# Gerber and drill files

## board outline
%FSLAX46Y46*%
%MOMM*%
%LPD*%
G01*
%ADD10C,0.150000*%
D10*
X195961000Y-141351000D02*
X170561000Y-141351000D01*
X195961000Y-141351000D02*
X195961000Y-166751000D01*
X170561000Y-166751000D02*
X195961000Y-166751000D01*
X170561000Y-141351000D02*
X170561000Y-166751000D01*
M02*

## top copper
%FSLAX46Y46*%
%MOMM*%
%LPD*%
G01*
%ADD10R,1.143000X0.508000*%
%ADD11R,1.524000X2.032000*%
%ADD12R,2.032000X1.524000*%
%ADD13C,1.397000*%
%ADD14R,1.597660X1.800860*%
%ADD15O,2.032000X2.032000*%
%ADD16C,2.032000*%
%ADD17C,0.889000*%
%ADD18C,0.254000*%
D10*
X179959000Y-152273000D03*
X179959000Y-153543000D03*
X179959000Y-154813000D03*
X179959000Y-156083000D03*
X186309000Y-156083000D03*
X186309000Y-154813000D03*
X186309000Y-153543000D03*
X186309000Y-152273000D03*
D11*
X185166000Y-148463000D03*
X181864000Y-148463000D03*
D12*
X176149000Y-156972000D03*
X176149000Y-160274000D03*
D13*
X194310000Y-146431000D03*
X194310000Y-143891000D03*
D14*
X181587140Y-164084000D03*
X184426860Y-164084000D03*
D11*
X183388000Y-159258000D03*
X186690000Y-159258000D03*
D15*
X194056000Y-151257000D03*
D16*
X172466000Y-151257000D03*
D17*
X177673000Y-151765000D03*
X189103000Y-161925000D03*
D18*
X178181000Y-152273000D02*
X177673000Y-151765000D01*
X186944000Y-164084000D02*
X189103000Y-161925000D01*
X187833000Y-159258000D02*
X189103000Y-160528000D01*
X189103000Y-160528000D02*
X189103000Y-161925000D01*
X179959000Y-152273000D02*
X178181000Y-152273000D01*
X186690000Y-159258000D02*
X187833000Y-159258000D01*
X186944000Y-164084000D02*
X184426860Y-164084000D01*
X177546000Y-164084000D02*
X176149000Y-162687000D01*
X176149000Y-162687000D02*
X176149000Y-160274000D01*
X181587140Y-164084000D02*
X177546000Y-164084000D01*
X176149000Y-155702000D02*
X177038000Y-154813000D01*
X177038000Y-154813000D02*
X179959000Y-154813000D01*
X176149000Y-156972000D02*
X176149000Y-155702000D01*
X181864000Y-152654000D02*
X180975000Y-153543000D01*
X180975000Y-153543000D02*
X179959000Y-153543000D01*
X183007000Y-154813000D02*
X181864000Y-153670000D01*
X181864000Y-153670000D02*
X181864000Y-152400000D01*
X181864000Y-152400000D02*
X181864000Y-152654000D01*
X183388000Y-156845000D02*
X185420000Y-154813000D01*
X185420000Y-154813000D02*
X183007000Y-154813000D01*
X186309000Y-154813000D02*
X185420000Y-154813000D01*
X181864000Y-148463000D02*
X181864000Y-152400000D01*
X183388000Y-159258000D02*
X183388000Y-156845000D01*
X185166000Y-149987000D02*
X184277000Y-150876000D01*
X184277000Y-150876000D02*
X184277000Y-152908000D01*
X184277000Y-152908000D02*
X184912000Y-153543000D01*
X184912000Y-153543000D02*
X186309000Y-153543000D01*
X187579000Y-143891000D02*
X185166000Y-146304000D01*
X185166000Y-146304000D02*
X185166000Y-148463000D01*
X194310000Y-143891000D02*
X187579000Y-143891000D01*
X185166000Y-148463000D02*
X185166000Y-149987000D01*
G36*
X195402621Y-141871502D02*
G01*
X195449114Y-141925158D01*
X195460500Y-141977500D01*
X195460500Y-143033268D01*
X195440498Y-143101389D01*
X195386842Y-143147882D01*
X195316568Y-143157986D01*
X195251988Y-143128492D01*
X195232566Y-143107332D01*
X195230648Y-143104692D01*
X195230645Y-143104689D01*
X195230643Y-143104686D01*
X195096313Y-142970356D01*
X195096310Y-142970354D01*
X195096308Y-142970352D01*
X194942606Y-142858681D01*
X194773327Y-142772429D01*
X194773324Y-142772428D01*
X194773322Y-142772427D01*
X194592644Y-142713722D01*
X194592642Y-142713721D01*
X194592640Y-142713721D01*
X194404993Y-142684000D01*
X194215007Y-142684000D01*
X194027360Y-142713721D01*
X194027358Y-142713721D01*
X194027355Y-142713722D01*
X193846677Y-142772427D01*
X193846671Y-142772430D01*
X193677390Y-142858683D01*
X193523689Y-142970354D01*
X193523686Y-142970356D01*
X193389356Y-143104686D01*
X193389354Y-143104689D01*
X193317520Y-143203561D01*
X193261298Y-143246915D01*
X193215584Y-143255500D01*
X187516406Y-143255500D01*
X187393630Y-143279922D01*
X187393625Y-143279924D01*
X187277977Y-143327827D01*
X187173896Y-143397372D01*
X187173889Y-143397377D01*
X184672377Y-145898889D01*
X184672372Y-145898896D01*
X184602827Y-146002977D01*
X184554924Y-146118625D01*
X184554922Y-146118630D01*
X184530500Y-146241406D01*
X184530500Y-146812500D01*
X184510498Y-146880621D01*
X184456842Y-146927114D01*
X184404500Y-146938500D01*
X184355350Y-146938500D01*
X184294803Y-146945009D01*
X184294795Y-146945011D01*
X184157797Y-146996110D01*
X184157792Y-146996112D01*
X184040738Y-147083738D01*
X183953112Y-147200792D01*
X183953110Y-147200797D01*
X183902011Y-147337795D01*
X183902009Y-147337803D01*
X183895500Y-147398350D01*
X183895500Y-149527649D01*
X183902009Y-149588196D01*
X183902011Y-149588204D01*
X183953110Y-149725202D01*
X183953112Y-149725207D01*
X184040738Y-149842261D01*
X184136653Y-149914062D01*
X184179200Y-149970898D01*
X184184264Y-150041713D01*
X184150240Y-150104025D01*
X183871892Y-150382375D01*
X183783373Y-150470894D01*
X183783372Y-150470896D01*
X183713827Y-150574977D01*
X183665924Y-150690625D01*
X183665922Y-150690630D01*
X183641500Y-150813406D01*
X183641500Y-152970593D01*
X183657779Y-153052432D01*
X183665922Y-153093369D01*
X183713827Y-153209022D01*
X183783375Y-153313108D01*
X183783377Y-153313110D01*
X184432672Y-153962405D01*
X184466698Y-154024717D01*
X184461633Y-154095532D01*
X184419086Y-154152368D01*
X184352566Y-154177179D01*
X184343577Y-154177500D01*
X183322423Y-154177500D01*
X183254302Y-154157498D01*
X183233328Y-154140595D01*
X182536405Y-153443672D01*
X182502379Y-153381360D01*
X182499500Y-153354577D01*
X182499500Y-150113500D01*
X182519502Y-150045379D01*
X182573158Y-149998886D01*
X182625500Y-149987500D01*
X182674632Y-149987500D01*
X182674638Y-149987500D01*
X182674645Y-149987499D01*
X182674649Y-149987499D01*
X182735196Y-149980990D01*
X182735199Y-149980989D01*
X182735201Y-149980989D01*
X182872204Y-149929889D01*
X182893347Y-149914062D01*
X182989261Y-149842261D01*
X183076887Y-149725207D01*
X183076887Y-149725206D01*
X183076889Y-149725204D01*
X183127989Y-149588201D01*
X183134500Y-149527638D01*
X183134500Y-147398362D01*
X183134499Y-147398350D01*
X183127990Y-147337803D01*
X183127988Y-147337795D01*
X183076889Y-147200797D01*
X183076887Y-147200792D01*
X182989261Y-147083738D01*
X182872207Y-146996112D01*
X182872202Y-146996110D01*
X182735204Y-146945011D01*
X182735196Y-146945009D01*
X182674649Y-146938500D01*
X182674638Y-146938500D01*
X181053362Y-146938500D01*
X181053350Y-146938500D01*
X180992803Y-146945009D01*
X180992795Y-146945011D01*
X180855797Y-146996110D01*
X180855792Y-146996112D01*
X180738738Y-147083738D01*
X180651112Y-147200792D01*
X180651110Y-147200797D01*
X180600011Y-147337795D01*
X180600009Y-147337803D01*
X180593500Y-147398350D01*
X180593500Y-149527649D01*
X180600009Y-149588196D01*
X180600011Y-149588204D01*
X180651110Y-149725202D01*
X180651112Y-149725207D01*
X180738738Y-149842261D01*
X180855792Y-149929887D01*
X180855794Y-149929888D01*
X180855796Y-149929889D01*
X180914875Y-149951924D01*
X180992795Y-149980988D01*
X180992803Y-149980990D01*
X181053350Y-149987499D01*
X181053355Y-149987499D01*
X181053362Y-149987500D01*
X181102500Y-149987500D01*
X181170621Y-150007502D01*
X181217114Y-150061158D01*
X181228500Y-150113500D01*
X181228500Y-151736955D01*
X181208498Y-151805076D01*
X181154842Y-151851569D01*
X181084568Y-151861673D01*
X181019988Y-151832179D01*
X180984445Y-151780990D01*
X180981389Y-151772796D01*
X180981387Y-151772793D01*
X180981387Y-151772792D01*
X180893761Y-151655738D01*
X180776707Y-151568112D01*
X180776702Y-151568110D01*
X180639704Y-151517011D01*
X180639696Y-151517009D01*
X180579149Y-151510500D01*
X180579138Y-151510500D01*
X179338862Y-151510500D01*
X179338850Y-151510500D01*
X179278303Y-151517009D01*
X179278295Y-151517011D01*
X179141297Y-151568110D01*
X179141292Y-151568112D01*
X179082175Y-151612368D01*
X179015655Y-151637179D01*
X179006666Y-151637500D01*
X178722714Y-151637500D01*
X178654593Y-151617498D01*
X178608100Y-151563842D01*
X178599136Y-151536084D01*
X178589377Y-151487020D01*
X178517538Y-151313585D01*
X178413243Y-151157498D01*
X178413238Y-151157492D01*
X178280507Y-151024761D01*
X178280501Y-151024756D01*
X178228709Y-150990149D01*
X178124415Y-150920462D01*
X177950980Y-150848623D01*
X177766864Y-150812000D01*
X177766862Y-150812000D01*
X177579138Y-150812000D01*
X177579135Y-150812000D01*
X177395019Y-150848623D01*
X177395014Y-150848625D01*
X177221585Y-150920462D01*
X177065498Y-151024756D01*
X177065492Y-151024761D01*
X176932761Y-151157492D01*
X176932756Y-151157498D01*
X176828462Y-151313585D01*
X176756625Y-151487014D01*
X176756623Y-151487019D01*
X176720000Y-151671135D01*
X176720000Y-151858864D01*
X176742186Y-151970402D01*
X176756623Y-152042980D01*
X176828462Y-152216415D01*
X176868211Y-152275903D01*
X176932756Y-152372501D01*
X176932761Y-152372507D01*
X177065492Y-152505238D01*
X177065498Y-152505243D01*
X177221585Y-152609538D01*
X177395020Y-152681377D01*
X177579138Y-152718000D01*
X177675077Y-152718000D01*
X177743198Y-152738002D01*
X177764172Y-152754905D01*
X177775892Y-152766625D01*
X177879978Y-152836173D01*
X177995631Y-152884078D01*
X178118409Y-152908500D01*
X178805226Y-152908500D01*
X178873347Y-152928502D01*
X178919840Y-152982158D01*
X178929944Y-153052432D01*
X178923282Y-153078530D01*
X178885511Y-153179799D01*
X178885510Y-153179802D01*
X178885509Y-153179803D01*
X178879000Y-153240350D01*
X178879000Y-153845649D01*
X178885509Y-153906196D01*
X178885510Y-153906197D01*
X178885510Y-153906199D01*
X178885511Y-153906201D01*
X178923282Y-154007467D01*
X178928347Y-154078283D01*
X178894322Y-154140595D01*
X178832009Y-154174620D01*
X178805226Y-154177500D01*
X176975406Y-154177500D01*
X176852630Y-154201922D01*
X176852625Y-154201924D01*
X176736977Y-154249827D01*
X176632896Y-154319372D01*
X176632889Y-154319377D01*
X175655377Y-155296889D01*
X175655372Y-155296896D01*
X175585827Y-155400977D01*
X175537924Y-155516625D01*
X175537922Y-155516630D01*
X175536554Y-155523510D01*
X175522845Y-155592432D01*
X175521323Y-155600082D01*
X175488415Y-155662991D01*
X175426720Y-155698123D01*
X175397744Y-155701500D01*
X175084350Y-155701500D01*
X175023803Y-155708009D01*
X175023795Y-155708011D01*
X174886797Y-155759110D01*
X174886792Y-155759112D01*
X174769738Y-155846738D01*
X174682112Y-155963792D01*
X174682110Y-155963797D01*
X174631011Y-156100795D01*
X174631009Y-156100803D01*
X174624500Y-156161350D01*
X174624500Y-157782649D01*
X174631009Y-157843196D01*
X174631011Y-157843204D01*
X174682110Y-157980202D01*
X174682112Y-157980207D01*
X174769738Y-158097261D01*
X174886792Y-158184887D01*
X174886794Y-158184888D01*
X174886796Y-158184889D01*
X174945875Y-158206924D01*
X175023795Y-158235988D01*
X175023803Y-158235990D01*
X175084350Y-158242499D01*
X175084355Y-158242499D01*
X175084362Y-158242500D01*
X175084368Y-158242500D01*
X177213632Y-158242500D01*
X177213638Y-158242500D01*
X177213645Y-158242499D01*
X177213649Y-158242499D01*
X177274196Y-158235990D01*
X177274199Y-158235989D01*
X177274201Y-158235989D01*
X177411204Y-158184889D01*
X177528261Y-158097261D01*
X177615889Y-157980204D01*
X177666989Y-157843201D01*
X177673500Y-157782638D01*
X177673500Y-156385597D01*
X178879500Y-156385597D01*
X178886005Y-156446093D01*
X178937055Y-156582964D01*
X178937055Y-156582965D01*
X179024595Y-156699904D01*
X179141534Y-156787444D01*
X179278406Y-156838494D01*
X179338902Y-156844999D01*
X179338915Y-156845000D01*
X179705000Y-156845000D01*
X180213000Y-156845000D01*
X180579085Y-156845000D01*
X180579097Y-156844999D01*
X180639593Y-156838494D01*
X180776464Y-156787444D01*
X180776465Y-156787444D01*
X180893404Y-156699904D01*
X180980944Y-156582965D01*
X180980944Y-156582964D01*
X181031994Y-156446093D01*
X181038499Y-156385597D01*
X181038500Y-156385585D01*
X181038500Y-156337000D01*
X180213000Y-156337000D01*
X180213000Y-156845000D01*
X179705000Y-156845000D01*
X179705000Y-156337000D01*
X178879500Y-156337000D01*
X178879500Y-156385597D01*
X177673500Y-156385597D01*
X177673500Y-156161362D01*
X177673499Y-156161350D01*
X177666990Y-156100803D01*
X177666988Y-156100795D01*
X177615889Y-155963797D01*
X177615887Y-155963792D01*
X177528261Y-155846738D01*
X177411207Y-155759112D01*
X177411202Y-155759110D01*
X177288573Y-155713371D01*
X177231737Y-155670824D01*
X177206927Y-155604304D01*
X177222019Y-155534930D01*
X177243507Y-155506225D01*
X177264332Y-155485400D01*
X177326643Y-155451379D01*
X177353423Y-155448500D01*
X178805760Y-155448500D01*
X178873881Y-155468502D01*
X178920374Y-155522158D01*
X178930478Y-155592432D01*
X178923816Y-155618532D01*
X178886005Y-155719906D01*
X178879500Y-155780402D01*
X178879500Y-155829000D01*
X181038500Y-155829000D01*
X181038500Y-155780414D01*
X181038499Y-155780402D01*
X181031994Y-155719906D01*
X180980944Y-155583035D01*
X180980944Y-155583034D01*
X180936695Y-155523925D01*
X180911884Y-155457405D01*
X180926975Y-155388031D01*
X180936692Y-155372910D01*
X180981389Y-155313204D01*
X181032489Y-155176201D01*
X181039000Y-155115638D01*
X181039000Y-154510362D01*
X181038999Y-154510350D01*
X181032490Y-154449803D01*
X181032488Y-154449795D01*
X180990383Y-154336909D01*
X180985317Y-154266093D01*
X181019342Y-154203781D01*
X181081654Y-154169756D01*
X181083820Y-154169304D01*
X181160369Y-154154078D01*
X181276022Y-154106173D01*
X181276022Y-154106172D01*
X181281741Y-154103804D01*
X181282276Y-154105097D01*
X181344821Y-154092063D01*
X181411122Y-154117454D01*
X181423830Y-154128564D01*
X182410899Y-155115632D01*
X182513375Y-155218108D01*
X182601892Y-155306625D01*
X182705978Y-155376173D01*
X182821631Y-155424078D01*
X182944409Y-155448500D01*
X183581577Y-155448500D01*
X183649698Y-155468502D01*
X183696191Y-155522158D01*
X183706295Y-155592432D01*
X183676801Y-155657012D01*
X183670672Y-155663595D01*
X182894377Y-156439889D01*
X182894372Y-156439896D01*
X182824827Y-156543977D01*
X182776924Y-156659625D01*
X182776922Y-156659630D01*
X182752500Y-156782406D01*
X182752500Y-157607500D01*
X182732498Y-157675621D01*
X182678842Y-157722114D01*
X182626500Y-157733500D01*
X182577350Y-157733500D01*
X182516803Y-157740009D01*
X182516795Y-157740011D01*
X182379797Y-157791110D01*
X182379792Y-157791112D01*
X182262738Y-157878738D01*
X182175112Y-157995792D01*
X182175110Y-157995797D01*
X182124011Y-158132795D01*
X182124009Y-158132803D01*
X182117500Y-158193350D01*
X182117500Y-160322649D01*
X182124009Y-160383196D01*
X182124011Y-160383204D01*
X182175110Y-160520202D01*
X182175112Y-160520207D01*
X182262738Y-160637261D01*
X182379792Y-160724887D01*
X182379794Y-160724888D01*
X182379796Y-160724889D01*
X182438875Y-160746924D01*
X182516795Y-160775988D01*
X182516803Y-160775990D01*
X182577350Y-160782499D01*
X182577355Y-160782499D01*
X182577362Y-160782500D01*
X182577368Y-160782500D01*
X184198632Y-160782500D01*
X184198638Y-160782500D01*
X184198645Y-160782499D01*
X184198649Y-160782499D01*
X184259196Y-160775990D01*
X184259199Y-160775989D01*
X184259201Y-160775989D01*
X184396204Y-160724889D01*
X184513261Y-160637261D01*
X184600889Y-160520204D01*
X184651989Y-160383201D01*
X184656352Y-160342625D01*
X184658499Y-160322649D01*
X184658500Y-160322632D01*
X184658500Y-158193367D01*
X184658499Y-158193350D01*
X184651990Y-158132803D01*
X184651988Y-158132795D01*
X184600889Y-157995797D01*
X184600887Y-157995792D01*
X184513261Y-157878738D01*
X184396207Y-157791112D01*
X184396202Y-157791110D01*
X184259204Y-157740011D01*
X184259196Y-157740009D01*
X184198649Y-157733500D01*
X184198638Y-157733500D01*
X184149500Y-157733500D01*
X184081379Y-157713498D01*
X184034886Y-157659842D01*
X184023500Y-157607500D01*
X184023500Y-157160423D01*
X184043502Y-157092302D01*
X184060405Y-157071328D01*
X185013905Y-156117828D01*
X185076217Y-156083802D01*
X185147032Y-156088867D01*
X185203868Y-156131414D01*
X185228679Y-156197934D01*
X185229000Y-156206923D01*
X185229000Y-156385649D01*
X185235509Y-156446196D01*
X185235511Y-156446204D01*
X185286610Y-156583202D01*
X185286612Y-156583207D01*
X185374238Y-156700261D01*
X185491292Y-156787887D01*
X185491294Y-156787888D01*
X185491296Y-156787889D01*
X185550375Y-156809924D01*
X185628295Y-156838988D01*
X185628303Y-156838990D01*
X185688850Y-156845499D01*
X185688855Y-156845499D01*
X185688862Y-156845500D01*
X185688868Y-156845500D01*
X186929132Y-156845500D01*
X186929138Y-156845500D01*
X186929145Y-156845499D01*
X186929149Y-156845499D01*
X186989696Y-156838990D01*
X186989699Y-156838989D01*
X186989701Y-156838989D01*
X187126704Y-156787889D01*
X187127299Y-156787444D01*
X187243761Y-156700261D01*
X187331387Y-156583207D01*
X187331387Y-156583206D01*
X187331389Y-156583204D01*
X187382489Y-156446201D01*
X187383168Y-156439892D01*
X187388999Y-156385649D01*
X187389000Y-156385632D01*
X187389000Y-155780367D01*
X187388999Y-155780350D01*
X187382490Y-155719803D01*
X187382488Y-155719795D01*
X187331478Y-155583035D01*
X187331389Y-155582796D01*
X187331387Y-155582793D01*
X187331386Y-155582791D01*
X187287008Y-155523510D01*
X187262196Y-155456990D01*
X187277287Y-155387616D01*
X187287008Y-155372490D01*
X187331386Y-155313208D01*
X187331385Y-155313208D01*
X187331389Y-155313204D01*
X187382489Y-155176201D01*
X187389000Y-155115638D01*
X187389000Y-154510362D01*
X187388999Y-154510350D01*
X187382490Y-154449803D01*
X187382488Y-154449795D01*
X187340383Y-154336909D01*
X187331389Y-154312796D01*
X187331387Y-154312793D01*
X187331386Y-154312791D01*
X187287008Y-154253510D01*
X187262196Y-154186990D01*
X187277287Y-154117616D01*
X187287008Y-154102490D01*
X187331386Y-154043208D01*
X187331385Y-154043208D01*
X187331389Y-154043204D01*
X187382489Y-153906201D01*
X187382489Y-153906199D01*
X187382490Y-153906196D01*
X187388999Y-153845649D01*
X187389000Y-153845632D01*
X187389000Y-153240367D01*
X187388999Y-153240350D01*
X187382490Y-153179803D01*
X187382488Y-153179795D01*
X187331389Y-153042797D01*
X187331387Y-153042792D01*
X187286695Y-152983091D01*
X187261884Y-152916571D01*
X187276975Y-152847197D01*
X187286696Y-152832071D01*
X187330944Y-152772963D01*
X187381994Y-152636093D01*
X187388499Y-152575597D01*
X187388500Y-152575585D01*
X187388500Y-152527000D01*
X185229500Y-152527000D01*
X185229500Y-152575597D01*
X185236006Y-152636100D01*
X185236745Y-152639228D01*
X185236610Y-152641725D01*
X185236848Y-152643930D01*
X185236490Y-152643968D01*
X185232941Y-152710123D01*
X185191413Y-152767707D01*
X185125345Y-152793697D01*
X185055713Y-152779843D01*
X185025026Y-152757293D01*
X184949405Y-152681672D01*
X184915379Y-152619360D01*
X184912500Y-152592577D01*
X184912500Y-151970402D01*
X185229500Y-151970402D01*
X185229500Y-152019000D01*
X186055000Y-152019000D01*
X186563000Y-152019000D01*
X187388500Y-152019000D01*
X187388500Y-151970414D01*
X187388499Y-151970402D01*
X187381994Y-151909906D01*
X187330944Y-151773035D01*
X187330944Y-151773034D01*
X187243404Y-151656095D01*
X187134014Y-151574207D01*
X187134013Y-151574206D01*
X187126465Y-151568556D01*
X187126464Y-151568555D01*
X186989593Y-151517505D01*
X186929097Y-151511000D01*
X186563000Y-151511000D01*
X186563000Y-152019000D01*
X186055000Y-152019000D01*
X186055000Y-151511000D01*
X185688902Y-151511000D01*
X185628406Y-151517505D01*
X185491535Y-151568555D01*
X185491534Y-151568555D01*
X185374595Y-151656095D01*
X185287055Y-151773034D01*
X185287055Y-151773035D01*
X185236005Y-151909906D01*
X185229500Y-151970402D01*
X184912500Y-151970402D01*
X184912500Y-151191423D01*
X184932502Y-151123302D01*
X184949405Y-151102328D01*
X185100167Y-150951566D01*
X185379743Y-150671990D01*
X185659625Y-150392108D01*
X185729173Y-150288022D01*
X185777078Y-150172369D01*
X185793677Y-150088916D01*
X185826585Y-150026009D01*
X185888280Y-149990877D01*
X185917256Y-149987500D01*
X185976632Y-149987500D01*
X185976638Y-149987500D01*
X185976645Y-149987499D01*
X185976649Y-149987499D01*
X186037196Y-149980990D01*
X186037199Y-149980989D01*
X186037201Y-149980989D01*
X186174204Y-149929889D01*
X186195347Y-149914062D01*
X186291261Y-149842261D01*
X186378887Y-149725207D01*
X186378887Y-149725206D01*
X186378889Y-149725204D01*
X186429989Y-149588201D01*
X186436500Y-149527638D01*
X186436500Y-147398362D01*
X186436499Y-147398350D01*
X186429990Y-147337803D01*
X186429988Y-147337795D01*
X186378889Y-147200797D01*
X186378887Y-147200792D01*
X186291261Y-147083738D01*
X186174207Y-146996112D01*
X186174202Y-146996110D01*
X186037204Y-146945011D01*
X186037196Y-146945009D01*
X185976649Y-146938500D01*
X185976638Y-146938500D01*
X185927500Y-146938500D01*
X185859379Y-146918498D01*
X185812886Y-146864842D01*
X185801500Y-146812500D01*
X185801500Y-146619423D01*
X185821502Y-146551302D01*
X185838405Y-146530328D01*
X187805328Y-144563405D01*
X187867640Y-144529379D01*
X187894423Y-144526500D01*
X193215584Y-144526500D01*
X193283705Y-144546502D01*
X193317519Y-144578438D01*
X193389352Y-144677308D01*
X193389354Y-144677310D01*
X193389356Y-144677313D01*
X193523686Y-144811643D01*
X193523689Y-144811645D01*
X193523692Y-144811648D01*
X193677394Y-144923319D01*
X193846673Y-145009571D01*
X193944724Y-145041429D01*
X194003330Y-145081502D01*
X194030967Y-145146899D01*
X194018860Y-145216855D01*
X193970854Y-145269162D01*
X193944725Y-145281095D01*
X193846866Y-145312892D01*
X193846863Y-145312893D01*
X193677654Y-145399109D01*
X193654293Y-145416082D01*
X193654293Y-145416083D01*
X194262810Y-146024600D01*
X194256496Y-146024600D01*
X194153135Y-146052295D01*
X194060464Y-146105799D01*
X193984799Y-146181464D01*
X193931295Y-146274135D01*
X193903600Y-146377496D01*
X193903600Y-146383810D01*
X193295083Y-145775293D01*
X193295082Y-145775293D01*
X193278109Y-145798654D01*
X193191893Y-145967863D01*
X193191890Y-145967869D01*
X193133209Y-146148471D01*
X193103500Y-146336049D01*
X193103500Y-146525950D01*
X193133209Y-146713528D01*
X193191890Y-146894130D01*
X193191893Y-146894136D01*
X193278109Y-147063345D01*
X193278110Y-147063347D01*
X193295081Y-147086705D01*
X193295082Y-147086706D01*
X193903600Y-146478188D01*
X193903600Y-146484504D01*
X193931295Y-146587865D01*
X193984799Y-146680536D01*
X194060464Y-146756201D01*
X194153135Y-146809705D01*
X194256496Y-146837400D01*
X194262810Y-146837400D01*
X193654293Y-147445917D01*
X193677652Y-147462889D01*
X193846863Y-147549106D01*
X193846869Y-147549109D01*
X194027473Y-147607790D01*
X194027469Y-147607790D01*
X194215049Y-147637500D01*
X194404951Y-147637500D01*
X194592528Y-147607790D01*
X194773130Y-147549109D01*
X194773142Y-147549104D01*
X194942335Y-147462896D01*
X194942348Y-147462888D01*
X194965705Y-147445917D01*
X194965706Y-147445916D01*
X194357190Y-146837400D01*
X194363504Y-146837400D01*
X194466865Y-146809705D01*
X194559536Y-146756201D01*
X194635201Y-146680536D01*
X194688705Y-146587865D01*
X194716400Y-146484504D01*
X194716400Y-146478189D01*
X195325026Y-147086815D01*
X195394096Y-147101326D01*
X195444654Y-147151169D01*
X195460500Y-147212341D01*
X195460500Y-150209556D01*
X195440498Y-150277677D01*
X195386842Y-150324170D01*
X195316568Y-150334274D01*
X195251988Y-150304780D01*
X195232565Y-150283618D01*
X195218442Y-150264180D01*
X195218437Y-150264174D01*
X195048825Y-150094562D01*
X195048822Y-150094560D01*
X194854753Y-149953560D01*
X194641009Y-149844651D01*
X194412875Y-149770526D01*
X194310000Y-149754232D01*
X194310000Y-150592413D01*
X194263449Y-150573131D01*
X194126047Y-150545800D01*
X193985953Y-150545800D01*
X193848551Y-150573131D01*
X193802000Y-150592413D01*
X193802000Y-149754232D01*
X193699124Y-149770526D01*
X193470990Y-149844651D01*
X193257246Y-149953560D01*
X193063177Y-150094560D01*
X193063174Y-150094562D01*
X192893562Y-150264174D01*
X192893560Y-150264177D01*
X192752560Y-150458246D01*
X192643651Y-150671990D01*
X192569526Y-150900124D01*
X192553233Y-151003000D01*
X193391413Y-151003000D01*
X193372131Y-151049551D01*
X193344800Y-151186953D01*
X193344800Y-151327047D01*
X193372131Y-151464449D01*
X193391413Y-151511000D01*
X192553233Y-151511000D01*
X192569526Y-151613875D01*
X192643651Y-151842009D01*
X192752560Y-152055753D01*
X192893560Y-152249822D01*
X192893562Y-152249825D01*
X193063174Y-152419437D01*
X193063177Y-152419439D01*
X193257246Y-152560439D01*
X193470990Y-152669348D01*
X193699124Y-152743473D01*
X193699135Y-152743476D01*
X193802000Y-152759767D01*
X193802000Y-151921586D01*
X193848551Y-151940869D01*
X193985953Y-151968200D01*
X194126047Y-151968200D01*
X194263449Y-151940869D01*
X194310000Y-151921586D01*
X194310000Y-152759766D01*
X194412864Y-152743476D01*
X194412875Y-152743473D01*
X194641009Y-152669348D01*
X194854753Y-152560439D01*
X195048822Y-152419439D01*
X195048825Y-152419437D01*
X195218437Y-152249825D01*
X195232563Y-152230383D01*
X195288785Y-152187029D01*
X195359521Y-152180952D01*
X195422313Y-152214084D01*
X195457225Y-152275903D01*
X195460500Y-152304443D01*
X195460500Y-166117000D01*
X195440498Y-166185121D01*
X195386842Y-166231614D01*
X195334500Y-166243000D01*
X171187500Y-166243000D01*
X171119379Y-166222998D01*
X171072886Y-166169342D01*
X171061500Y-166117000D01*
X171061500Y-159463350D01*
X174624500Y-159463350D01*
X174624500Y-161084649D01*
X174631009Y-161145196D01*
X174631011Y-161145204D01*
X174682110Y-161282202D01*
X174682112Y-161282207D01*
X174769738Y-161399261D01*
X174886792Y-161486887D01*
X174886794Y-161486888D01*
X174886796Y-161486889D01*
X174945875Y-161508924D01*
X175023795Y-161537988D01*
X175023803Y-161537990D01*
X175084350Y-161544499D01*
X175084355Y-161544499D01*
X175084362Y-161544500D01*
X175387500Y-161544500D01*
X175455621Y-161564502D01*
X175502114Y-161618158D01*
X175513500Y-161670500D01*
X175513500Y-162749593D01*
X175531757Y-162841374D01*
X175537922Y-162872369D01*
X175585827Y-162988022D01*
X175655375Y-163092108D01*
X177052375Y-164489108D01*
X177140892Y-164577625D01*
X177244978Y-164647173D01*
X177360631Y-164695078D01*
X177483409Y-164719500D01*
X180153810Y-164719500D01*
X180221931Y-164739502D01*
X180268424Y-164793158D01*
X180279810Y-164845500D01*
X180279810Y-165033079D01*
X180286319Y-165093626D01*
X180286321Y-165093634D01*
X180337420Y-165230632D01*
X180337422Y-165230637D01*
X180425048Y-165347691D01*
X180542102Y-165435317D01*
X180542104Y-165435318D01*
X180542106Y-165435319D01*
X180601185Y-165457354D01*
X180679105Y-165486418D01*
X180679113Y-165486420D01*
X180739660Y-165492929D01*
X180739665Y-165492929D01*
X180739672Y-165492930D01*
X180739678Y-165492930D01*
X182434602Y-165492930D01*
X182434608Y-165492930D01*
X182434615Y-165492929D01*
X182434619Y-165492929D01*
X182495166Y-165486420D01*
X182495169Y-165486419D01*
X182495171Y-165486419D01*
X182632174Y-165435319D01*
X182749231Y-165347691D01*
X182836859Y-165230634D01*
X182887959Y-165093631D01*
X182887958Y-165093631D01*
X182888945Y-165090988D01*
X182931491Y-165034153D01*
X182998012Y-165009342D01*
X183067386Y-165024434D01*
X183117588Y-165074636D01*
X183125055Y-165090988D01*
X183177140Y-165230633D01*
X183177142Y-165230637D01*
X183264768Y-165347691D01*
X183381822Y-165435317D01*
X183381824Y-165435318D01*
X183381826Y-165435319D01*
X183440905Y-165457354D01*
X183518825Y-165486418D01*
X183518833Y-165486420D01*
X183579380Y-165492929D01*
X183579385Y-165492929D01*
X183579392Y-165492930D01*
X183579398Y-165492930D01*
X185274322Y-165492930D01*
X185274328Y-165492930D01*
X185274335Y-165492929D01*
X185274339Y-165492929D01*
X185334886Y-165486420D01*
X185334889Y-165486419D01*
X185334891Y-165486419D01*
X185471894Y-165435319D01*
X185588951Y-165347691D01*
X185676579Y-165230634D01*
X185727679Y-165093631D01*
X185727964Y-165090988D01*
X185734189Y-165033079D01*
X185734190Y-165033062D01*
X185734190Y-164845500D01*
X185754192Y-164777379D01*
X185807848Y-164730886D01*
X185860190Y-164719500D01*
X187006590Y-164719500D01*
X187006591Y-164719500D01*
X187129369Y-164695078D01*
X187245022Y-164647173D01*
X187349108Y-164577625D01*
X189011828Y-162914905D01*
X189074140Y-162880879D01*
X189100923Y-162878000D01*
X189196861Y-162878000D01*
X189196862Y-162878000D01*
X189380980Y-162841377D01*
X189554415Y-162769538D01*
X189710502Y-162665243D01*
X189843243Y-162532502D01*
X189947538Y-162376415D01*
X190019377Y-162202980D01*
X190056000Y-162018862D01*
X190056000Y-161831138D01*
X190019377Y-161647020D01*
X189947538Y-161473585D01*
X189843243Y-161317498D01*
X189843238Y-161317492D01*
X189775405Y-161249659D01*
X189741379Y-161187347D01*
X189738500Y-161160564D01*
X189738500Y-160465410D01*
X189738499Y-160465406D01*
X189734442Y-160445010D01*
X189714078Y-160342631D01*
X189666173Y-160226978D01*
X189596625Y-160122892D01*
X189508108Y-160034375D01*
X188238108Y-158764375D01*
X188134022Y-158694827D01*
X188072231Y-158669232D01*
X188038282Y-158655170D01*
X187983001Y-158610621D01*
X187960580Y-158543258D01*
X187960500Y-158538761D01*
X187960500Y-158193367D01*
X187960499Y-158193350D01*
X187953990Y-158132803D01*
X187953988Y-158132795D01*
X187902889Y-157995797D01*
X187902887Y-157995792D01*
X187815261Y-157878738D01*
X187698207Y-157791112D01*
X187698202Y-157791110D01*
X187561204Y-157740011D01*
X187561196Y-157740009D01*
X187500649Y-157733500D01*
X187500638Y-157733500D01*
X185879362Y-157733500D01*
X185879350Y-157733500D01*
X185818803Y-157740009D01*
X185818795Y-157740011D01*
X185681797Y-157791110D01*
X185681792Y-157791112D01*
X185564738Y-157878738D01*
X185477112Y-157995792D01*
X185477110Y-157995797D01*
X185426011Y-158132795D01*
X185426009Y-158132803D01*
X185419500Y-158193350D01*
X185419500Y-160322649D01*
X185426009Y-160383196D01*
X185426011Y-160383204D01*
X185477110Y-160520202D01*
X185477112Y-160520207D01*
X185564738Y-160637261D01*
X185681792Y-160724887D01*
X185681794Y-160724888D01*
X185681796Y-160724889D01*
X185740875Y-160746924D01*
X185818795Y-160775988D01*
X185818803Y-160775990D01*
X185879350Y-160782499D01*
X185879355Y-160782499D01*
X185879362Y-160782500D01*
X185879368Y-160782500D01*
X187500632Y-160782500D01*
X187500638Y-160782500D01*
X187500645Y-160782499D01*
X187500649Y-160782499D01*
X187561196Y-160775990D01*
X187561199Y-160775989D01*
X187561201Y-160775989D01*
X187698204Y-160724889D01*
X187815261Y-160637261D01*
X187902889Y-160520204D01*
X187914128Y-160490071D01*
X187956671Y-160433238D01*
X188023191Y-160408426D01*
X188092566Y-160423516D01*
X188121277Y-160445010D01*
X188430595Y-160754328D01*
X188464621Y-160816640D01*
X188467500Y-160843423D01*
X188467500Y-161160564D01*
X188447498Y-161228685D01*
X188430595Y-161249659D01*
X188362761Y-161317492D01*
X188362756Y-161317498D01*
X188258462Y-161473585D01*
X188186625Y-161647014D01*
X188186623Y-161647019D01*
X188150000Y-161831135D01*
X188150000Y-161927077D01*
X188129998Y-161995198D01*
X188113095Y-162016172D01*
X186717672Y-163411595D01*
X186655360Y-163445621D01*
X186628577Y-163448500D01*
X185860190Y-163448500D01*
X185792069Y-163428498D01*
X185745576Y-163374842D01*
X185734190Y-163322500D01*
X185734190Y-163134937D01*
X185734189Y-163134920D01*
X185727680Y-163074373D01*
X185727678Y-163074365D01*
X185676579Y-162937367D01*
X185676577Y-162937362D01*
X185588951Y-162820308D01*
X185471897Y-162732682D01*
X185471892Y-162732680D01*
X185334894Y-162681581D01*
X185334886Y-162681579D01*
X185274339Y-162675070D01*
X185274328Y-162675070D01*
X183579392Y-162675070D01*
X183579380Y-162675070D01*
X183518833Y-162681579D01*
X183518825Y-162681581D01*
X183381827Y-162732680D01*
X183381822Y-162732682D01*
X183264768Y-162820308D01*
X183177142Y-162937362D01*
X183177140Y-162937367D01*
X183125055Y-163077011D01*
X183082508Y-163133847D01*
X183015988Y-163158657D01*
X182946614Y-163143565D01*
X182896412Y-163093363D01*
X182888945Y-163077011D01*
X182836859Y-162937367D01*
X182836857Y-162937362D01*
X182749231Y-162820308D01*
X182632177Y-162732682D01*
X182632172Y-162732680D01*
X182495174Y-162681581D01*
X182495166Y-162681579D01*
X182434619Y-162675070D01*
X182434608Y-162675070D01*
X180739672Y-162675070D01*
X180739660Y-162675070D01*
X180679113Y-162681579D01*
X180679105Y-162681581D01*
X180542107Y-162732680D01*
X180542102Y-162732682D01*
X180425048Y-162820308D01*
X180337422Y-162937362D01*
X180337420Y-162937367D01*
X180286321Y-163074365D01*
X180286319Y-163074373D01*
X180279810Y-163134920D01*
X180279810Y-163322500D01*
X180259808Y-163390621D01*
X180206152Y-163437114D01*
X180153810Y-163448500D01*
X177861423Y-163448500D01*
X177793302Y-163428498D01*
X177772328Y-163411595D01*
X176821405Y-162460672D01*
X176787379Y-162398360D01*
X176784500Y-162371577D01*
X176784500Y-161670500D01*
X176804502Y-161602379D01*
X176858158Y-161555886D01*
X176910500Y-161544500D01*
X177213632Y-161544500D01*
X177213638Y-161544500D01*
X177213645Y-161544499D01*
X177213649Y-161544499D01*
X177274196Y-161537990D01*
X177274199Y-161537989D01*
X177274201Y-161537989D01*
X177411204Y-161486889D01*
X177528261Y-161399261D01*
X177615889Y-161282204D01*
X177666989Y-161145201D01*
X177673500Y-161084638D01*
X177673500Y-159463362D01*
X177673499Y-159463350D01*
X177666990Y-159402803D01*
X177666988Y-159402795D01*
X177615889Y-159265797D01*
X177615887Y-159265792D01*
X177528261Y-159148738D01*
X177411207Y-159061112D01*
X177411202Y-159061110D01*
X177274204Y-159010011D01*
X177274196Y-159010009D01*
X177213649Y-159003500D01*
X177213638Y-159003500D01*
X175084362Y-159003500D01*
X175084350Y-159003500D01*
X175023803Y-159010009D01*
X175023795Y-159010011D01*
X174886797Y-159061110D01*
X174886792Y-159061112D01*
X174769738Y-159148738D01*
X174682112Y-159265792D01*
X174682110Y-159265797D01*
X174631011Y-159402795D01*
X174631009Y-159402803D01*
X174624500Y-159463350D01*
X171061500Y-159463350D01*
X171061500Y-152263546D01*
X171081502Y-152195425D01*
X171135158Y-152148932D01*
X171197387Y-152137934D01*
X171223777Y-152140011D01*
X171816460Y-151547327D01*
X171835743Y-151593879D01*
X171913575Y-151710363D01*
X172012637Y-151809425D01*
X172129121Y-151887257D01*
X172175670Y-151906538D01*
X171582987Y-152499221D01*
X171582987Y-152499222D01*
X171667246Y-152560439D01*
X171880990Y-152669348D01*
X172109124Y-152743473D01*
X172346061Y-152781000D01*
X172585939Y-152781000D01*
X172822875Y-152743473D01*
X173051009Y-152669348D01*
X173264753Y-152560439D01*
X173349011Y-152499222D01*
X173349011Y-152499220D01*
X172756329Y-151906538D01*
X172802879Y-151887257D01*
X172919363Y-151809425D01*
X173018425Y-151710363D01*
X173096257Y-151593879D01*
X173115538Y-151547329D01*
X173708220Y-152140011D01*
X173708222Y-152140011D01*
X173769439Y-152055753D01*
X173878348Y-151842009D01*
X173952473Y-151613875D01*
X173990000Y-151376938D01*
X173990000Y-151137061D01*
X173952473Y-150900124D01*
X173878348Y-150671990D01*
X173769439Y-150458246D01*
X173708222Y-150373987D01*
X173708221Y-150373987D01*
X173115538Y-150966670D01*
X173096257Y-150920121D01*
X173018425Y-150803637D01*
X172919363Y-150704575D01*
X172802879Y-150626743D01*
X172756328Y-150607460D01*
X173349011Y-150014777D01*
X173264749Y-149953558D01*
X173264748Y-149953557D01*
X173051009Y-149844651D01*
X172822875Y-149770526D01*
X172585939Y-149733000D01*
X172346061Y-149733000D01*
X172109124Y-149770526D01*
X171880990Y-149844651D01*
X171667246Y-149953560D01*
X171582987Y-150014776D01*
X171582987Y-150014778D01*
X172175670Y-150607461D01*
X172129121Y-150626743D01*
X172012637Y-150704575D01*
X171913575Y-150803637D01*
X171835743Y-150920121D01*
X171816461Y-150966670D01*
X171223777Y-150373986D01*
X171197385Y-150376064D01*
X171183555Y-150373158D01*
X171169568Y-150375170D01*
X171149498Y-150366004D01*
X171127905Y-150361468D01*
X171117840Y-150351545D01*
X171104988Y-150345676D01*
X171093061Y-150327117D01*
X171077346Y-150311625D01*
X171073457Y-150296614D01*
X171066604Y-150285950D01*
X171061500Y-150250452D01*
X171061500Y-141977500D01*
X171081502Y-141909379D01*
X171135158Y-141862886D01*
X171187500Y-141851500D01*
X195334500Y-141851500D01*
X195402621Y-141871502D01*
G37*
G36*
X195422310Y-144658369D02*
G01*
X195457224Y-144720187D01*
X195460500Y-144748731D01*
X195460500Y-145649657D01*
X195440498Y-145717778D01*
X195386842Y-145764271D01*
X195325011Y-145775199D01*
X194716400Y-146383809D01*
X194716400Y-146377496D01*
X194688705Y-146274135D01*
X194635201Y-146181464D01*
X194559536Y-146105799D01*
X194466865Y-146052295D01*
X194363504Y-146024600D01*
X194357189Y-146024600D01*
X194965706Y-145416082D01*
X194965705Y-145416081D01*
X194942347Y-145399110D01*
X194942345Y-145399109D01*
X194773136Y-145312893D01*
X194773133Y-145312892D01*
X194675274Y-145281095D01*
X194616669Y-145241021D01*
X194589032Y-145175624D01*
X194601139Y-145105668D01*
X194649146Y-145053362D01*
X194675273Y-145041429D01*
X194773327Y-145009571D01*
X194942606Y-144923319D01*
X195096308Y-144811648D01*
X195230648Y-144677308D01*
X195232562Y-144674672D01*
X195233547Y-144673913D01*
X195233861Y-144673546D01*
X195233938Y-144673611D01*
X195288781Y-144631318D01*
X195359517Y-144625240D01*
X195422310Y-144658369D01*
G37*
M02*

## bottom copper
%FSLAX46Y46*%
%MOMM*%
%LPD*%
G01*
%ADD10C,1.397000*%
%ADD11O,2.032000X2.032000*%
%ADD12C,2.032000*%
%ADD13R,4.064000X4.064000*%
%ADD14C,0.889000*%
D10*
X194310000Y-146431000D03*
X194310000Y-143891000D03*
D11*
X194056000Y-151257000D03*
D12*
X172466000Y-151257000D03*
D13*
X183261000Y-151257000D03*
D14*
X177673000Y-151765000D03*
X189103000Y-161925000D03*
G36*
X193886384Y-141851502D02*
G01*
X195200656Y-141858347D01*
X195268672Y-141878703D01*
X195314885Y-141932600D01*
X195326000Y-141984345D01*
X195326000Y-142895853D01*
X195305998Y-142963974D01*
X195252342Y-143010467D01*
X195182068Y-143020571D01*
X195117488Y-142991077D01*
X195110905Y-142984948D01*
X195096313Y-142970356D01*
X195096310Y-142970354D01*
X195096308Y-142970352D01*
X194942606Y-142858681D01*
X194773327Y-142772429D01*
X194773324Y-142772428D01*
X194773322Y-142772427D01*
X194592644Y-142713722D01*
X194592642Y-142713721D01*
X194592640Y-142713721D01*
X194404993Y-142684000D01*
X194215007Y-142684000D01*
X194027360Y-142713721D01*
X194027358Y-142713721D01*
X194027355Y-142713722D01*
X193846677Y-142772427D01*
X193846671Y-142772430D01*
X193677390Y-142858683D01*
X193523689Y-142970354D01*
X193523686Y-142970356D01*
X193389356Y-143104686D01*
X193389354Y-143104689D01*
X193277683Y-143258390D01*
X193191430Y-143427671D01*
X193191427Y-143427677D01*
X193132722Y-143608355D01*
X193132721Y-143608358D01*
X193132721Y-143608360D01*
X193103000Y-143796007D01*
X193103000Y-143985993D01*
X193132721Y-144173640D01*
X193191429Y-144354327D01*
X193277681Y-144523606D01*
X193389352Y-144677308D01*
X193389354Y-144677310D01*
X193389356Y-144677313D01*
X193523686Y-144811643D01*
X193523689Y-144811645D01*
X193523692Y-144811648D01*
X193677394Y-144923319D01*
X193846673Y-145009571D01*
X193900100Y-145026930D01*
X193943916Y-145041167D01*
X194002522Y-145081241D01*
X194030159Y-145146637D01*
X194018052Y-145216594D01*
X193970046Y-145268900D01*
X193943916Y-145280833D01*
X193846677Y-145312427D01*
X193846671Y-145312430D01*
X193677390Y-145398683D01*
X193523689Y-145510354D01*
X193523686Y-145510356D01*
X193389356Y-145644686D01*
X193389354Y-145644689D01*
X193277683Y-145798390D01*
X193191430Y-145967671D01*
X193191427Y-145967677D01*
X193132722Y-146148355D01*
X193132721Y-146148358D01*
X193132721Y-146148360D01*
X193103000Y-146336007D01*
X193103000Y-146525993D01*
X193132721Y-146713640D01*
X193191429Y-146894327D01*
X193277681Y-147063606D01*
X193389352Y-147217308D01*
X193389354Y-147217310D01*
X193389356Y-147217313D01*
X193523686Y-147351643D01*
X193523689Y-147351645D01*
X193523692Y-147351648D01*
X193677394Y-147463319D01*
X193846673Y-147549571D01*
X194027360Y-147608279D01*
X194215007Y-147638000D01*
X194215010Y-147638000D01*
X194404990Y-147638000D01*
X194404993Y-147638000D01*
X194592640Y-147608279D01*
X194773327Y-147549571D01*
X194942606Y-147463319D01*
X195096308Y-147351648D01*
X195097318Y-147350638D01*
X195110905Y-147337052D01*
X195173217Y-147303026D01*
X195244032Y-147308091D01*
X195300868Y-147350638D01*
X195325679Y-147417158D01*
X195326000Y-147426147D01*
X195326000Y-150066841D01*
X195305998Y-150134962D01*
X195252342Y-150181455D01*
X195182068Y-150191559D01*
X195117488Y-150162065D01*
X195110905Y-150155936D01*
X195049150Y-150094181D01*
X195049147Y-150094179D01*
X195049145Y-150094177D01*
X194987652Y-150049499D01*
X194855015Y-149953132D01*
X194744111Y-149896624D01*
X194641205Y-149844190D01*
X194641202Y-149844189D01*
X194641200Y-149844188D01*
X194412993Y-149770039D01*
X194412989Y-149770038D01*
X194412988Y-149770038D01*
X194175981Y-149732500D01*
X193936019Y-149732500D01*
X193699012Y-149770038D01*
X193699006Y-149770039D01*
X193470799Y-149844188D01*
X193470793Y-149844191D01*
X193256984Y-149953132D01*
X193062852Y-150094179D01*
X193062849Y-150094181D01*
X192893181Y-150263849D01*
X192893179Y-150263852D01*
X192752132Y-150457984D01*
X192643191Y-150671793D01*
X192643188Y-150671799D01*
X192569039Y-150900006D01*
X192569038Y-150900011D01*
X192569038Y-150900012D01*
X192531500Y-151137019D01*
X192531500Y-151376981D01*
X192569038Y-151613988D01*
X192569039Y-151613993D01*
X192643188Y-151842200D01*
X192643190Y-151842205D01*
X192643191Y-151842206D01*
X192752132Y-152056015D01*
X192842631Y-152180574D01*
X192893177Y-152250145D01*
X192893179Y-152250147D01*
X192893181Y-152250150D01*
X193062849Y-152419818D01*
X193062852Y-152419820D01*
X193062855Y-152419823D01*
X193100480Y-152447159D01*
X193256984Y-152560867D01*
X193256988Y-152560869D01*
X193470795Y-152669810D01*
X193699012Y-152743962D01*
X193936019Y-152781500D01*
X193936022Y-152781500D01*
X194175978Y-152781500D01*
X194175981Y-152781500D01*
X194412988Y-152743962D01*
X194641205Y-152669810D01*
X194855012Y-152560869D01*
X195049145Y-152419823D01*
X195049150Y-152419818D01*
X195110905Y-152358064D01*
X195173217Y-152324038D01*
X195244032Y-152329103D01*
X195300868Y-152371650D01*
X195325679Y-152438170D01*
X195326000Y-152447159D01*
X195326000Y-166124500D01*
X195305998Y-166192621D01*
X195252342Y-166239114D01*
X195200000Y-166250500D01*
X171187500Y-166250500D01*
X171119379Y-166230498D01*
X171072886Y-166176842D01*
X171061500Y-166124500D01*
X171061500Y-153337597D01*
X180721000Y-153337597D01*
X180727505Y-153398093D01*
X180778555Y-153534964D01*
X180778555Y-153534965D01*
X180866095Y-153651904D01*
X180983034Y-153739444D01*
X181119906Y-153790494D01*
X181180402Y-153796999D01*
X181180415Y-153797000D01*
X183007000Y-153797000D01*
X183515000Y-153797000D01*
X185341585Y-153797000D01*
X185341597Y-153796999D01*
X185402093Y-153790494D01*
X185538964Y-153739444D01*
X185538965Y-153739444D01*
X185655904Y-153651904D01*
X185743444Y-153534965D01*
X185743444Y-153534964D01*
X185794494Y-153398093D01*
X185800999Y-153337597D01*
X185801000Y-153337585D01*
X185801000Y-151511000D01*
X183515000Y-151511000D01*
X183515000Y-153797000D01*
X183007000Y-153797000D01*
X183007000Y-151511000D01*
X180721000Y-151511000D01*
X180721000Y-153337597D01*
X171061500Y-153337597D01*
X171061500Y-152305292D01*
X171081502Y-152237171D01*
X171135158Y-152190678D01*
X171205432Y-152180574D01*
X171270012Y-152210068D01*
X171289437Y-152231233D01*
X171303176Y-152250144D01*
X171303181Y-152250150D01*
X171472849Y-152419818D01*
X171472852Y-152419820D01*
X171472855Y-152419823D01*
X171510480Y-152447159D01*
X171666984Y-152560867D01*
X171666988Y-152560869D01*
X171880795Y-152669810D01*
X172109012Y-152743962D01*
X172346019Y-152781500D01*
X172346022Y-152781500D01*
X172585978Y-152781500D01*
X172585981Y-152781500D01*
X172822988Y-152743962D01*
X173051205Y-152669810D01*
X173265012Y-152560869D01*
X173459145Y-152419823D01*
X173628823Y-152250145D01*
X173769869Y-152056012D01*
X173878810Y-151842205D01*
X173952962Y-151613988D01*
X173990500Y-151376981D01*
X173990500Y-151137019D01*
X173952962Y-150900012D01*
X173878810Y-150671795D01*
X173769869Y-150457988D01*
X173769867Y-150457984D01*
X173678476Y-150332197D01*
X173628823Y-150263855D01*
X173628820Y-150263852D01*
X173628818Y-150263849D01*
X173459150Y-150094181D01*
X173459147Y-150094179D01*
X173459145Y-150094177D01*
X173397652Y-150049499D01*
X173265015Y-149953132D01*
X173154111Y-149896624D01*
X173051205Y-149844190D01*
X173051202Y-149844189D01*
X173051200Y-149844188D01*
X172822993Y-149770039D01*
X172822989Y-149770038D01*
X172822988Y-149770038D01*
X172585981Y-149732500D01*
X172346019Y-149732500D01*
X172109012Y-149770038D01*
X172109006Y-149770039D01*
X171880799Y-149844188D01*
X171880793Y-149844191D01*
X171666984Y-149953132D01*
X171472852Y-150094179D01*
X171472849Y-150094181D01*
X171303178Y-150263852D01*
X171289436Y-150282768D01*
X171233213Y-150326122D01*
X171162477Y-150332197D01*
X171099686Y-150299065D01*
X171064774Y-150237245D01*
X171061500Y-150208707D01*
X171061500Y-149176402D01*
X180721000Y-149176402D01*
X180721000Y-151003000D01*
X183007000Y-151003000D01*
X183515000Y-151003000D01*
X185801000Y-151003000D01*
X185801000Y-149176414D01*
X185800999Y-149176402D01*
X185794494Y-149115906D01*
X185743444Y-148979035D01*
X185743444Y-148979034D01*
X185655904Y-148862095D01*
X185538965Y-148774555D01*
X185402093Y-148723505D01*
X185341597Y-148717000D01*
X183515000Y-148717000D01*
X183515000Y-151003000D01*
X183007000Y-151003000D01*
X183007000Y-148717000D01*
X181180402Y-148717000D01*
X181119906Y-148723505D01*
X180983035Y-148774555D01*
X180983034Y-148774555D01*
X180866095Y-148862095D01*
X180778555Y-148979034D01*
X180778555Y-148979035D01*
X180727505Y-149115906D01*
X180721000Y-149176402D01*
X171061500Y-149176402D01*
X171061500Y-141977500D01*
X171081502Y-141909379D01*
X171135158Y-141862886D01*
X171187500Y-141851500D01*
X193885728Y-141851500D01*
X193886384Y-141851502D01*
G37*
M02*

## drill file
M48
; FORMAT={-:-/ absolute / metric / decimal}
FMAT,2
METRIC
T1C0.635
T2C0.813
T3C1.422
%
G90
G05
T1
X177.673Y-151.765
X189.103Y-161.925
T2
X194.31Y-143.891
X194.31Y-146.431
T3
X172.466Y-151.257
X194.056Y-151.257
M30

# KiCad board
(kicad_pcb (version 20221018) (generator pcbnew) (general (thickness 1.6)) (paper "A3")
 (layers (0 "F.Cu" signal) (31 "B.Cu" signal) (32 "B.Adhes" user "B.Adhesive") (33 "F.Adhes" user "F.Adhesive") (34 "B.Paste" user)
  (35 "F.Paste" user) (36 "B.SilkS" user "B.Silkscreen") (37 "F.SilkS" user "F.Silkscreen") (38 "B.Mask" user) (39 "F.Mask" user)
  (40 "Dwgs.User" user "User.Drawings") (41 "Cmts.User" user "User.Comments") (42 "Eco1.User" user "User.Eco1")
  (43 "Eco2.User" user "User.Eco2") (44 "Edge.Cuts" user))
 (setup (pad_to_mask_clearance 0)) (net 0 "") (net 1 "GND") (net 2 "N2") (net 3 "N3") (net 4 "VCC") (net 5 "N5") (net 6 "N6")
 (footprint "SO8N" (layer "F.Cu") (at 183.134 154.178 -90)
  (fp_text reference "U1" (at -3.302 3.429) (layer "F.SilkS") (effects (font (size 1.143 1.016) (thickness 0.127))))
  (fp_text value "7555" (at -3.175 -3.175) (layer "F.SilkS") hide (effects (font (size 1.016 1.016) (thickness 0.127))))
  (pad "1" smd rect (at -1.905 3.175 270) (size 0.508 1.143) (layers "F.Cu" "F.Paste" "F.Mask") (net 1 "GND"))
  (pad "2" smd rect (at -0.635 3.175 270) (size 0.508 1.143) (layers "F.Cu" "F.Paste" "F.Mask") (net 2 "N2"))
  (pad "3" smd rect (at 0.635 3.175 270) (size 0.508 1.143) (layers "F.Cu" "F.Paste" "F.Mask") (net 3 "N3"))
  (pad "4" smd rect (at 1.905 3.175 270) (size 0.508 1.143) (layers "F.Cu" "F.Paste" "F.Mask") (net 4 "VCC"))
  (pad "5" smd rect (at 1.905 -3.175 270) (size 0.508 1.143) (layers "F.Cu" "F.Paste" "F.Mask"))
  (pad "6" smd rect (at 0.635 -3.175 270) (size 0.508 1.143) (layers "F.Cu" "F.Paste" "F.Mask") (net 2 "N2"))
  (pad "7" smd rect (at -0.635 -3.175 270) (size 0.508 1.143) (layers "F.Cu" "F.Paste" "F.Mask") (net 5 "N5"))
  (pad "8" smd rect (at -1.905 -3.175 270) (size 0.508 1.143) (layers "F.Cu" "F.Paste" "F.Mask") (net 4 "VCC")))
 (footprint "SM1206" (layer "F.Cu") (at 183.515 148.463 180)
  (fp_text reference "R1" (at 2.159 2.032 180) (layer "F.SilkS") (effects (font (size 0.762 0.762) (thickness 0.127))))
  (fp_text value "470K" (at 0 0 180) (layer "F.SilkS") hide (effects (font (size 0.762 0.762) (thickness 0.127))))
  (pad "1" smd rect (at -1.651 0 180) (size 1.524 2.032) (layers "F.Cu" "F.Paste" "F.Mask") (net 5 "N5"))
  (pad "2" smd rect (at 1.651 0 180) (size 1.524 2.032) (layers "F.Cu" "F.Paste" "F.Mask") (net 2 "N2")))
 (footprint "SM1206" (layer "F.Cu") (at 176.149 158.623 -90)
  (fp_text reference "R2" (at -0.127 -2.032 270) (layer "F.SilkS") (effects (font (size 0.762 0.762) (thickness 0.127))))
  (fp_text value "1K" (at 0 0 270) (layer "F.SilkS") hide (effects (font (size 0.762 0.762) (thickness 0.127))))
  (pad "1" smd rect (at -1.651 0 270) (size 1.524 2.032) (layers "F.Cu" "F.Paste" "F.Mask") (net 3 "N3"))
  (pad "2" smd rect (at 1.651 0 270) (size 1.524 2.032) (layers "F.Cu" "F.Paste" "F.Mask") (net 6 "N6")))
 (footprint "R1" (layer "F.Cu") (at 194.31 145.161 90)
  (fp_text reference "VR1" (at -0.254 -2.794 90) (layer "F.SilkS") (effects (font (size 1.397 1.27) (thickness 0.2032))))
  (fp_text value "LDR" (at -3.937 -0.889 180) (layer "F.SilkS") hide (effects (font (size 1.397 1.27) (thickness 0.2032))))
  (pad "1" thru_hole circle (at -1.27 0 90) (size 1.397 1.397) (drill 0.812799) (layers "*.Cu" "*.Mask" "F.SilkS") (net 4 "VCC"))
  (pad "2" thru_hole circle (at 1.27 0 90) (size 1.397 1.397) (drill 0.812799) (layers "*.Cu" "*.Mask" "F.SilkS") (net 5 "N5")))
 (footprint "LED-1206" (layer "F.Cu") (at 183.007 164.084)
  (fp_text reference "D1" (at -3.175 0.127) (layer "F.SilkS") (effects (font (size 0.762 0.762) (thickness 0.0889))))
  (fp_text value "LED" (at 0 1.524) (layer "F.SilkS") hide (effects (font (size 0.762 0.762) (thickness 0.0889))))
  (pad "1" smd rect (at -1.41986 0) (size 1.59766 1.80086) (layers "F.Cu" "F.Paste" "F.Mask") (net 6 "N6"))
  (pad "2" smd rect (at 1.41986 0) (size 1.59766 1.80086) (layers "F.Cu" "F.Paste" "F.Mask") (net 1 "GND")))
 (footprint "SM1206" (layer "F.Cu") (at 185.039 159.258)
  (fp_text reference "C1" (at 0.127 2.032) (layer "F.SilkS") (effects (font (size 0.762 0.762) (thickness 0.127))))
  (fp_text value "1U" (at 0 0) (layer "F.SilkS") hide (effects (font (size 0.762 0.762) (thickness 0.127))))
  (pad "1" smd rect (at -1.651 0) (size 1.524 2.032) (layers "F.Cu" "F.Paste" "F.Mask") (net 2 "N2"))
  (pad "2" smd rect (at 1.651 0) (size 1.524 2.032) (layers "F.Cu" "F.Paste" "F.Mask") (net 1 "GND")))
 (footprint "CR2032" (layer "B.Cu") (at 183.261 151.257 180)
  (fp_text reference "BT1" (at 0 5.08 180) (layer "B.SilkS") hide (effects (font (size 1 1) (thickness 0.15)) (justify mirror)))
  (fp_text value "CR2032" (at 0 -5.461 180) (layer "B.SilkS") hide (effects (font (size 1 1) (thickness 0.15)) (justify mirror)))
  (pad "1" thru_hole oval (at -10.795 0 180) (size 2.032 2.032) (drill 1.4224) (layers "*.Cu" "*.Mask" "B.SilkS") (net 4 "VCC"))
  (pad "1" thru_hole circle (at 10.795 0 180) (size 2.032 2.032) (drill 1.4224) (layers "*.Cu" "*.Mask" "B.SilkS") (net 4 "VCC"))
  (pad "2" smd rect (at 0 0 180) (size 4.064 4.064) (layers "B.Cu" "B.Paste" "B.Mask") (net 1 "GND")))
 (gr_line (start 195.961 141.351) (end 170.561 141.351) (stroke (width 0.15) (type solid)) (layer "Edge.Cuts"))
 (gr_line (start 195.961 141.351) (end 195.961 166.751) (stroke (width 0.15) (type solid)) (layer "Edge.Cuts"))
 (gr_line (start 170.561 166.751) (end 195.961 166.751) (stroke (width 0.15) (type solid)) (layer "Edge.Cuts"))
 (gr_line (start 170.561 141.351) (end 170.561 166.751) (stroke (width 0.15) (type solid)) (layer "Edge.Cuts"))
 (segment (start 178.181 152.273) (end 177.673 151.765) (width 0.254) (layer "F.Cu") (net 1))
 (segment (start 186.944 164.084) (end 189.103 161.925) (width 0.254) (layer "F.Cu") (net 1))
 (segment (start 187.833 159.258) (end 189.103 160.528) (width 0.254) (layer "F.Cu") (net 1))
 (segment (start 189.103 160.528) (end 189.103 161.925) (width 0.254) (layer "F.Cu") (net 1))
 (segment (start 179.959 152.273) (end 178.181 152.273) (width 0.254) (layer "F.Cu") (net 1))
 (segment (start 186.69 159.258) (end 187.833 159.258) (width 0.254) (layer "F.Cu") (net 1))
 (segment (start 186.944 164.084) (end 184.42686 164.084) (width 0.254) (layer "F.Cu") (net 1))
 (via (at 177.673 151.765) (size 0.889) (drill 0.635) (layers "F.Cu" "B.Cu") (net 1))
 (via (at 189.103 161.925) (size 0.889) (drill 0.635) (layers "F.Cu" "B.Cu") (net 1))
 (segment (start 177.546 164.084) (end 176.149 162.687) (width 0.254) (layer "F.Cu") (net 6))
 (segment (start 176.149 162.687) (end 176.149 160.274) (width 0.254) (layer "F.Cu") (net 6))
 (segment (start 181.58714 164.084) (end 177.546 164.084) (width 0.254) (layer "F.Cu") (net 6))
 (segment (start 176.149 155.702) (end 177.038 154.813) (width 0.254) (layer "F.Cu") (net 3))
 (segment (start 177.038 154.813) (end 179.959 154.813) (width 0.254) (layer "F.Cu") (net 3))
 (segment (start 176.149 156.972) (end 176.149 155.702) (width 0.254) (layer "F.Cu") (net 3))
 (segment (start 181.864 152.654) (end 180.975 153.543) (width 0.254) (layer "F.Cu") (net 2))
 (segment (start 180.975 153.543) (end 179.959 153.543) (width 0.254) (layer "F.Cu") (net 2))
 (segment (start 183.007 154.813) (end 181.864 153.67) (width 0.254) (layer "F.Cu") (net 2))
 (segment (start 181.864 153.67) (end 181.864 152.4) (width 0.254) (layer "F.Cu") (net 2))
 (segment (start 181.864 152.4) (end 181.864 152.654) (width 0.254) (layer "F.Cu") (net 2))
 (segment (start 183.388 156.845) (end 185.42 154.813) (width 0.254) (layer "F.Cu") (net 2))
 (segment (start 185.42 154.813) (end 183.007 154.813) (width 0.254) (layer "F.Cu") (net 2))
 (segment (start 186.309 154.813) (end 185.42 154.813) (width 0.254) (layer "F.Cu") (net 2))
 (segment (start 181.864 148.463) (end 181.864 152.4) (width 0.254) (layer "F.Cu") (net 2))
 (segment (start 183.388 159.258) (end 183.388 156.845) (width 0.254) (layer "F.Cu") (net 2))
 (segment (start 185.166 149.987) (end 184.277 150.876) (width 0.254) (layer "F.Cu") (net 5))
 (segment (start 184.277 150.876) (end 184.277 152.908) (width 0.254) (layer "F.Cu") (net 5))
 (segment (start 184.277 152.908) (end 184.912 153.543) (width 0.254) (layer "F.Cu") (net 5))
 (segment (start 184.912 153.543) (end 186.309 153.543) (width 0.254) (layer "F.Cu") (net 5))
 (segment (start 187.579 143.891) (end 185.166 146.304) (width 0.254) (layer "F.Cu") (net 5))
 (segment (start 185.166 146.304) (end 185.166 148.463) (width 0.254) (layer "F.Cu") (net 5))
 (segment (start 194.31 143.891) (end 187.579 143.891) (width 0.254) (layer "F.Cu") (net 5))
 (segment (start 185.166 148.463) (end 185.166 149.987) (width 0.254) (layer "F.Cu") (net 5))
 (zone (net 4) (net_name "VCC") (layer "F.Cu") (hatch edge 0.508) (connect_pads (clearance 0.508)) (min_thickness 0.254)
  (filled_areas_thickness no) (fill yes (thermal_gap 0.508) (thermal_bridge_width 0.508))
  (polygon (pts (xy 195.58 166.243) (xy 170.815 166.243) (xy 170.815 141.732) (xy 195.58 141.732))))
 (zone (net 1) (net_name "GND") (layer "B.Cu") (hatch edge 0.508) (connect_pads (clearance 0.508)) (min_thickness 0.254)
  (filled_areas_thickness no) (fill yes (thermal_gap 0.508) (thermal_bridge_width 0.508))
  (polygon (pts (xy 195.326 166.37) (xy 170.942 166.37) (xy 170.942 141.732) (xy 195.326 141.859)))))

